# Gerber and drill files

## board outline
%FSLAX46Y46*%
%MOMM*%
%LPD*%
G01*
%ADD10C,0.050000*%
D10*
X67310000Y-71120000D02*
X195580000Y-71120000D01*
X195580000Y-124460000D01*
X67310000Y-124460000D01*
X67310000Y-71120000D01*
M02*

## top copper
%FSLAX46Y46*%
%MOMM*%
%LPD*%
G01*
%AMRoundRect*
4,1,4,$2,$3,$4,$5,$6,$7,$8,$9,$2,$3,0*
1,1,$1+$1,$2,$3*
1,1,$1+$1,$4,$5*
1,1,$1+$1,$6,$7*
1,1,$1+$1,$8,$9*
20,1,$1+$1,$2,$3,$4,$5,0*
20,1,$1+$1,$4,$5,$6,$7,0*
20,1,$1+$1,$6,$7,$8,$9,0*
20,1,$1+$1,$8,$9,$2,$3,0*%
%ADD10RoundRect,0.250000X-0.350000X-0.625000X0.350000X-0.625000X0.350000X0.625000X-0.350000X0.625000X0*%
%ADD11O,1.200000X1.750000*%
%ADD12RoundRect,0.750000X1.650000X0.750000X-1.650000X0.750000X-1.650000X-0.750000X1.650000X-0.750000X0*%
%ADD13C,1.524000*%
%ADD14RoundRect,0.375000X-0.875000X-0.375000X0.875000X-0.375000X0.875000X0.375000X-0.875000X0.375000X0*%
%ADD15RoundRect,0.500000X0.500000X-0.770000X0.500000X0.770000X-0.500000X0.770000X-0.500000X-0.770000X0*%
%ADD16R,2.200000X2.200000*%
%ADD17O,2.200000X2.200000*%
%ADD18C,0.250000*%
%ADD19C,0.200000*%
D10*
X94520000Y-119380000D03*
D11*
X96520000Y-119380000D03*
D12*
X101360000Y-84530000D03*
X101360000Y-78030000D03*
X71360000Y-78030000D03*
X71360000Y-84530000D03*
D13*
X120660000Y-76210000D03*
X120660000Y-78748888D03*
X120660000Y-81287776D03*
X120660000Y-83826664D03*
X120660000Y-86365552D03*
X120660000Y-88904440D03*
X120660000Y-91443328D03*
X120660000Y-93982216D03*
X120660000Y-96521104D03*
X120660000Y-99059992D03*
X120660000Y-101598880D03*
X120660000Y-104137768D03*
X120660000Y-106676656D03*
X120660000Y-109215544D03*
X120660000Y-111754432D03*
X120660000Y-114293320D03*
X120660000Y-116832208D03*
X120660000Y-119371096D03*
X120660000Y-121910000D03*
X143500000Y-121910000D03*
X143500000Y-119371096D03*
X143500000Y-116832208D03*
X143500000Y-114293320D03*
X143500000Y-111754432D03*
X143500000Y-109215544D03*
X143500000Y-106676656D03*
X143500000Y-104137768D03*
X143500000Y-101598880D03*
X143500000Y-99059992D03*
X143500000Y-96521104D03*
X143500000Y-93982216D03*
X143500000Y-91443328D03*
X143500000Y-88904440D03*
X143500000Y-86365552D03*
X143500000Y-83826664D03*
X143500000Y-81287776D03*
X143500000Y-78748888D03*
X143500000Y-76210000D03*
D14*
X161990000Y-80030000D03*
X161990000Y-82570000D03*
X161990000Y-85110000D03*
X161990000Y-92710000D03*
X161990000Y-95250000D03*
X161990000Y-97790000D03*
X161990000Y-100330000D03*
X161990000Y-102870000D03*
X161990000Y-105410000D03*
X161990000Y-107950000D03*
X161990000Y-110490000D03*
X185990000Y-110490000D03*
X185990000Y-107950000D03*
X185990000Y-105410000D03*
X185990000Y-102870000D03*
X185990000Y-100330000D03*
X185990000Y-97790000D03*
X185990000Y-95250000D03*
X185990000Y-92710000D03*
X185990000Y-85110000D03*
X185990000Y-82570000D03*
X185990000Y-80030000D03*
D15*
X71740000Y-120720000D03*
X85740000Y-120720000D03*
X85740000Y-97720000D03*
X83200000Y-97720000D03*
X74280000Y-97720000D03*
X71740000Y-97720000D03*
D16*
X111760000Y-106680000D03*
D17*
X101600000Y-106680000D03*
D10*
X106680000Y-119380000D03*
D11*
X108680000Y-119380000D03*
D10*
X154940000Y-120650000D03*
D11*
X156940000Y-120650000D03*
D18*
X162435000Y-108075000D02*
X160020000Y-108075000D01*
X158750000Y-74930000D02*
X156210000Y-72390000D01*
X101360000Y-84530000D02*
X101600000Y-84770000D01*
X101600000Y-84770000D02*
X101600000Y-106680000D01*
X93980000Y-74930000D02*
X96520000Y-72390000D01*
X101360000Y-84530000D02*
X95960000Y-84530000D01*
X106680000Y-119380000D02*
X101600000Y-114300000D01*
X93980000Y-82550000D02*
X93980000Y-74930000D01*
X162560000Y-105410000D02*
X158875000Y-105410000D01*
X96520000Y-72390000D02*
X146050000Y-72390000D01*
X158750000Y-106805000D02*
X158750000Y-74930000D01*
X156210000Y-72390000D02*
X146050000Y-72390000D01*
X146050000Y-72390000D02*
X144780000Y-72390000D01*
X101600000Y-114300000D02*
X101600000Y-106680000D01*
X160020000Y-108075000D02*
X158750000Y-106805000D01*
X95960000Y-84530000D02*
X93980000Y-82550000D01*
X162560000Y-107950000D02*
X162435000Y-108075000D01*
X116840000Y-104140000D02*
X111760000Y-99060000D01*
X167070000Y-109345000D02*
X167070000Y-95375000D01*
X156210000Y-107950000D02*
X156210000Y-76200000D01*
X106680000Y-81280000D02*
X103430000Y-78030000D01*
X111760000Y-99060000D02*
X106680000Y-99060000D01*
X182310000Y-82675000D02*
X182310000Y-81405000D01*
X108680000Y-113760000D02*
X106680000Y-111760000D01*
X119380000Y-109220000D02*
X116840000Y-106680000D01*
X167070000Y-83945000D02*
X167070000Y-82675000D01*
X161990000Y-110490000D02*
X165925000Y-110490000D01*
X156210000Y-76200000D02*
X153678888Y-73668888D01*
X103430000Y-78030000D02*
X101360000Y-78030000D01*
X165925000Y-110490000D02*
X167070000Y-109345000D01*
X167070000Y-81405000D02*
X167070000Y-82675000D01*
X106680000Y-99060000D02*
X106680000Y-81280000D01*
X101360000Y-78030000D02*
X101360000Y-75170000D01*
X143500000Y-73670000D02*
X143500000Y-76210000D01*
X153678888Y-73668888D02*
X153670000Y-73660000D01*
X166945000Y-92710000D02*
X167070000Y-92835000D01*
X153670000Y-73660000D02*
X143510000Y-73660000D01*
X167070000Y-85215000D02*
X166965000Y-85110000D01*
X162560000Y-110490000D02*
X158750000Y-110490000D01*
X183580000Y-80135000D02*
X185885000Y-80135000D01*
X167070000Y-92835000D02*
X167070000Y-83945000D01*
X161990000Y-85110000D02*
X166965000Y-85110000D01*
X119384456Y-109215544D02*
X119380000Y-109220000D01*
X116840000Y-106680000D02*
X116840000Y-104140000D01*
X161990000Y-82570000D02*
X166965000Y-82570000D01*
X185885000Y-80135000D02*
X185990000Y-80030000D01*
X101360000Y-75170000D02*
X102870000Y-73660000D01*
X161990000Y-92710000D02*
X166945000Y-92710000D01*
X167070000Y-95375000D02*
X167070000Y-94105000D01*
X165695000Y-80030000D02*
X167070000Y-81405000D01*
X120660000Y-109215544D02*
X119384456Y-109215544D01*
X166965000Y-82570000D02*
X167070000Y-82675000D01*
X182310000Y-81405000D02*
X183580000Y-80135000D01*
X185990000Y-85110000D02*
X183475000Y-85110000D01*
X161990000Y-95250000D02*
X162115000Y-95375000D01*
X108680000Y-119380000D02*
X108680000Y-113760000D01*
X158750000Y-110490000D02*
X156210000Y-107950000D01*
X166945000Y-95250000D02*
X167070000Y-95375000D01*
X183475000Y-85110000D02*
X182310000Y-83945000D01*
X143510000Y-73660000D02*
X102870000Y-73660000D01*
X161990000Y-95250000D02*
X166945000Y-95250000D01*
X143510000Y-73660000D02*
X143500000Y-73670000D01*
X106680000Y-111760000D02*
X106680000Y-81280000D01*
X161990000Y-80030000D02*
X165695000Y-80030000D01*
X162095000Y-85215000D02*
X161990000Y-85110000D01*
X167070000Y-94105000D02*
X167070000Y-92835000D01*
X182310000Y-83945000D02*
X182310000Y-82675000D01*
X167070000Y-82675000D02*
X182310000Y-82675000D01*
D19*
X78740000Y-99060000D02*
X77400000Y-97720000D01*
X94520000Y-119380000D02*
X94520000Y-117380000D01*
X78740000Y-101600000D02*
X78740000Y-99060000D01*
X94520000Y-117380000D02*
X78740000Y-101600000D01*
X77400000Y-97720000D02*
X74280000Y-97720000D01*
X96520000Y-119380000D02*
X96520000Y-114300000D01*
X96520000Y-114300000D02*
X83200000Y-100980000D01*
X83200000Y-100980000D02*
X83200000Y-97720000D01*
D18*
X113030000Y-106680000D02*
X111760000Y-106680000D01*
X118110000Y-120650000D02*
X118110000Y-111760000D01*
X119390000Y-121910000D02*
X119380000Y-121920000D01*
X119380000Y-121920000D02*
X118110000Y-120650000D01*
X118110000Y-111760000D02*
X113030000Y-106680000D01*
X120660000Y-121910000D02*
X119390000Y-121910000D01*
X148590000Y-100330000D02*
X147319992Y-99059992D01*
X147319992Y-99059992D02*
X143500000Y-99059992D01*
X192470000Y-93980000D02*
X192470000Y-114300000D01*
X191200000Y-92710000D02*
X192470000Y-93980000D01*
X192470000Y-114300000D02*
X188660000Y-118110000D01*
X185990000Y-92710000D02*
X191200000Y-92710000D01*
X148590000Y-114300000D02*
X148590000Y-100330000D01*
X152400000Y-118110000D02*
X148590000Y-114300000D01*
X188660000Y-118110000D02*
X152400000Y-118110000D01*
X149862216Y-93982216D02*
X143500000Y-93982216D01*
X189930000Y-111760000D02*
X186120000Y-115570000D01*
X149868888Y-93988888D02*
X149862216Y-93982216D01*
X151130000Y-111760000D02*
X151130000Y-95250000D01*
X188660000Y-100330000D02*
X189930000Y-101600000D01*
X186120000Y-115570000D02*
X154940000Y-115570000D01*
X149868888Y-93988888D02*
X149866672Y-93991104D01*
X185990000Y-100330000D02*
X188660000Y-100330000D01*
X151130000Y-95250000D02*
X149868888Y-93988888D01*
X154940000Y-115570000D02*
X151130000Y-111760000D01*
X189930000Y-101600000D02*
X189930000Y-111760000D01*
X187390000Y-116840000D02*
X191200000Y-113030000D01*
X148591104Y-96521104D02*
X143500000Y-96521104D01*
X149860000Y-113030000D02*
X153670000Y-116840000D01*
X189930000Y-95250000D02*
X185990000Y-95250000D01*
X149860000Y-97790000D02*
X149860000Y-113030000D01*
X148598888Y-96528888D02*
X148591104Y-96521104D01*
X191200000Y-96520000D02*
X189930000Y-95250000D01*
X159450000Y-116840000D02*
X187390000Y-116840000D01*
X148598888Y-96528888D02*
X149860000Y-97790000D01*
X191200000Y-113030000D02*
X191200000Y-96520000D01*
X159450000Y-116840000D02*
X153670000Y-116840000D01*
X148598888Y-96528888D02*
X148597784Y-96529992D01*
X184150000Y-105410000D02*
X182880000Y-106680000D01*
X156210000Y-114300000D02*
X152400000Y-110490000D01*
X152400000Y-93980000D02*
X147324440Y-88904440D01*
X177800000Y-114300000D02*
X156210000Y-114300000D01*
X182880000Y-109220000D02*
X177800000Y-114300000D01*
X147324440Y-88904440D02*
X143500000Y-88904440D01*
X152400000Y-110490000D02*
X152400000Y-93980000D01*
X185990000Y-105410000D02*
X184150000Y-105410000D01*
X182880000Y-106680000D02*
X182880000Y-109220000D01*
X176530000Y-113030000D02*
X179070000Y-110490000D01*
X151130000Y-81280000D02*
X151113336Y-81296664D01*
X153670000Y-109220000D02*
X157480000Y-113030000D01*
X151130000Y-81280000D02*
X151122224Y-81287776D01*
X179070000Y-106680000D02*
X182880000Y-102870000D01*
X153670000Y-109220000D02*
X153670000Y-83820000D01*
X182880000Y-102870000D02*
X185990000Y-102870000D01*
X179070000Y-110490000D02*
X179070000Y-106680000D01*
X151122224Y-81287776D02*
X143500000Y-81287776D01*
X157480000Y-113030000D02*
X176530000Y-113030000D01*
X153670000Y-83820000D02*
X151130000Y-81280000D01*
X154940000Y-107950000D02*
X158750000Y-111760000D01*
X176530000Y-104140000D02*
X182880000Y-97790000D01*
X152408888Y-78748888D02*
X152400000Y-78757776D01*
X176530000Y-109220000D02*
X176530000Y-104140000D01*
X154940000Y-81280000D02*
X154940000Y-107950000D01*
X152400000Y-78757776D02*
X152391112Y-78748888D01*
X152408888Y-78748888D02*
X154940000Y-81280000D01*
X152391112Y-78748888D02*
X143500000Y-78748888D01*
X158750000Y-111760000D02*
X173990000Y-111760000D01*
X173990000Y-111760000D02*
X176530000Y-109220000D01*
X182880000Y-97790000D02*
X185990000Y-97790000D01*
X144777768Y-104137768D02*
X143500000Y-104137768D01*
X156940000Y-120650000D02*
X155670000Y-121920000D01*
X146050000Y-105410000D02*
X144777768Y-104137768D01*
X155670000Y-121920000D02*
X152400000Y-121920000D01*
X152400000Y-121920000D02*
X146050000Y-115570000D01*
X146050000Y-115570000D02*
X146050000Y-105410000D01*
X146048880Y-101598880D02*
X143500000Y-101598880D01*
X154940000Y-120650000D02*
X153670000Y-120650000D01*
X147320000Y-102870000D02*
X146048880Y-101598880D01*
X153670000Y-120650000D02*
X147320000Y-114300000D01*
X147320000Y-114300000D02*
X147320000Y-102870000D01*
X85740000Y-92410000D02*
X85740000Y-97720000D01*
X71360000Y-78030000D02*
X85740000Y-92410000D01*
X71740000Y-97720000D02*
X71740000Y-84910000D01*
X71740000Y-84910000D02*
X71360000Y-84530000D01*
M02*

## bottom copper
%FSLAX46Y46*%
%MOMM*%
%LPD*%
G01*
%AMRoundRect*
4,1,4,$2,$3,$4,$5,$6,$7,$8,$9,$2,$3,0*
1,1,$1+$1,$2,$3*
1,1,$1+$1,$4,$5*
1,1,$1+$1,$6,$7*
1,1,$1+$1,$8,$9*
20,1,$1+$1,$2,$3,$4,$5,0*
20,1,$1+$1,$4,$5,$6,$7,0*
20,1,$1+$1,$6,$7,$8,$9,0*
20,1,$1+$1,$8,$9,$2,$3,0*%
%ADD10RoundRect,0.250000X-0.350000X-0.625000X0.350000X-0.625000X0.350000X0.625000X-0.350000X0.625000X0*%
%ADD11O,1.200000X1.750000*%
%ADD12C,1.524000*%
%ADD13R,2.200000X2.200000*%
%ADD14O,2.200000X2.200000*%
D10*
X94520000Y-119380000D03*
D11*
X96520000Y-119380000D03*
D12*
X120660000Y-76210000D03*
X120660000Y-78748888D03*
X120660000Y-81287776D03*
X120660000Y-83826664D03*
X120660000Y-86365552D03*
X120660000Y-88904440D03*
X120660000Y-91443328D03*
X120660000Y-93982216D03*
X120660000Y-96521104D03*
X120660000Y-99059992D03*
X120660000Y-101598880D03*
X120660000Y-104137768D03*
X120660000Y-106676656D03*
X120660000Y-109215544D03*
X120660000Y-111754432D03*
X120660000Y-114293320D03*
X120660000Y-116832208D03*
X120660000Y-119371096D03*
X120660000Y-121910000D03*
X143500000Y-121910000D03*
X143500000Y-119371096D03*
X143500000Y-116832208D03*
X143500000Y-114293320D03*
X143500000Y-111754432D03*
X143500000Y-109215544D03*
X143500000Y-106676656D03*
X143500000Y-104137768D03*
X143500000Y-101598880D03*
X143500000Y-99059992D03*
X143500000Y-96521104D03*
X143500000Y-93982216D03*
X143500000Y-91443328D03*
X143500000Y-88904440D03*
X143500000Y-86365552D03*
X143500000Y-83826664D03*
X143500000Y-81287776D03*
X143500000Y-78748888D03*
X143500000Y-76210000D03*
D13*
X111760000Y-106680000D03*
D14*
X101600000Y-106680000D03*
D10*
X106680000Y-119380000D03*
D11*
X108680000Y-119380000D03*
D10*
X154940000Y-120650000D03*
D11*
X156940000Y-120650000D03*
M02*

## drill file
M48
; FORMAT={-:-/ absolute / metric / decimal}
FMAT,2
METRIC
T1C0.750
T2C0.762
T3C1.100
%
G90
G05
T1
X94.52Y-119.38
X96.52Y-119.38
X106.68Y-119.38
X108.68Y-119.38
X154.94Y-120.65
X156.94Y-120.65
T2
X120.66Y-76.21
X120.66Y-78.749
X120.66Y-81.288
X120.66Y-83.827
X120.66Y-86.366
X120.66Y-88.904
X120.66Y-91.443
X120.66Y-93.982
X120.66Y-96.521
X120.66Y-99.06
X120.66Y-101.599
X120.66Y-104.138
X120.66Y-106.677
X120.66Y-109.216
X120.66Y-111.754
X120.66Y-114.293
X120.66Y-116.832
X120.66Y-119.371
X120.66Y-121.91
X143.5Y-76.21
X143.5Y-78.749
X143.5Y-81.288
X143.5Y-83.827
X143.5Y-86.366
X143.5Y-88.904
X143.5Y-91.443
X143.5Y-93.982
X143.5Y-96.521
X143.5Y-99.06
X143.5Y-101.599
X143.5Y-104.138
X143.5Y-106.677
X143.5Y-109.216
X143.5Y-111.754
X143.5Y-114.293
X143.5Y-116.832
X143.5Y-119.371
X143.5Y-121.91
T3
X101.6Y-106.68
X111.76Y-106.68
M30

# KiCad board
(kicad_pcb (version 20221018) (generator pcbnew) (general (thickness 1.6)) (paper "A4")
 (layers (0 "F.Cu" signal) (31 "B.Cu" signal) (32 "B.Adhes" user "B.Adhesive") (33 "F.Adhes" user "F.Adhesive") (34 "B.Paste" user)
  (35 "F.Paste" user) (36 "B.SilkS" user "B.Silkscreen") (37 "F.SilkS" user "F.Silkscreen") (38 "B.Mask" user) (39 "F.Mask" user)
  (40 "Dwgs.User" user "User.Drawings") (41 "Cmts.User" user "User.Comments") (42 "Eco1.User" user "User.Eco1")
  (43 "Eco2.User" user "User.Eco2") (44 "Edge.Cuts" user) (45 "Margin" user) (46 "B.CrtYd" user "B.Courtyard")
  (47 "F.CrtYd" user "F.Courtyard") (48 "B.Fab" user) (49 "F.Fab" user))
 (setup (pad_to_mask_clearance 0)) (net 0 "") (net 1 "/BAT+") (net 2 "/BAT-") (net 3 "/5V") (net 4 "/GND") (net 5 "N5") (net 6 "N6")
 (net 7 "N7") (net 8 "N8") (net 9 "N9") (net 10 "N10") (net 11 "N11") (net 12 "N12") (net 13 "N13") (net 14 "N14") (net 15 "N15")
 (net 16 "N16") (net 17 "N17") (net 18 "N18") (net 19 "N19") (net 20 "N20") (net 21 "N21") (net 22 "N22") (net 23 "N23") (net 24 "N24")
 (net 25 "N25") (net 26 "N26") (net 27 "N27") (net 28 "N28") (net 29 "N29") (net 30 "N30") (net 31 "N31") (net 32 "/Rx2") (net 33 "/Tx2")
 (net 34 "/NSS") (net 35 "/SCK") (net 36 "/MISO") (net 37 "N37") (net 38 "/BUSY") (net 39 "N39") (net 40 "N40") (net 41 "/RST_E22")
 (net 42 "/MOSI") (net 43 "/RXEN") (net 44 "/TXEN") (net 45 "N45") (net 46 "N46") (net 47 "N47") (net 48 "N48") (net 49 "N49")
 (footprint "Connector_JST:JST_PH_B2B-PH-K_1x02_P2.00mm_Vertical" (layer "F.Cu") (at 94.52 119.38)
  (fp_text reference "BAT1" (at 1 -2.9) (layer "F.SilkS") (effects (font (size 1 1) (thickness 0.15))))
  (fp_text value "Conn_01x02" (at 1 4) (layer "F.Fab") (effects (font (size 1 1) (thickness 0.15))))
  (pad "1" thru_hole roundrect (at 0 0) (size 1.2 1.75) (drill 0.75) (layers "*.Cu" "*.Mask") (roundrect_rratio 0.208333) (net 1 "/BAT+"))
  (pad "2" thru_hole oval (at 2 0) (size 1.2 1.75) (drill 0.75) (layers "*.Cu" "*.Mask") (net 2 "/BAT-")))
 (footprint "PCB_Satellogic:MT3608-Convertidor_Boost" (layer "F.Cu") (at 86.36 81.28 180)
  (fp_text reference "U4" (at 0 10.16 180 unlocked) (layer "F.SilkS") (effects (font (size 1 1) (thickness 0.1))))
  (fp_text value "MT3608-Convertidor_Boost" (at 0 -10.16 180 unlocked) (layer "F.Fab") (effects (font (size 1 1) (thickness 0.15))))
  (pad "1" smd roundrect (at -15 -3.25 180) (size 4.8 3) (layers "F.Cu" "F.Paste" "F.Mask") (roundrect_rratio 0.25) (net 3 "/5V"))
  (pad "2" smd roundrect (at -15 3.25 180) (size 4.8 3) (layers "F.Cu" "F.Paste" "F.Mask") (roundrect_rratio 0.25) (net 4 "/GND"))
  (pad "3" smd roundrect (at 15 3.25 180) (size 4.8 3) (layers "F.Cu" "F.Paste" "F.Mask") (roundrect_rratio 0.25) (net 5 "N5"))
  (pad "4" smd roundrect (at 15 -3.25 180) (size 4.8 3) (layers "F.Cu" "F.Paste" "F.Mask") (roundrect_rratio 0.25) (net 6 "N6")))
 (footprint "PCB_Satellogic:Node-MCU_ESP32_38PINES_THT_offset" (layer "F.Cu") (at 132.08 99.06)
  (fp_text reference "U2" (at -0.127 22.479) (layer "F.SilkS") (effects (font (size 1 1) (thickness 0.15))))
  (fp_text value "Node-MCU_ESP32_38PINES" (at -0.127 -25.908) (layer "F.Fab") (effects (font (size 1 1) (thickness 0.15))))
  (pad "1" thru_hole circle (at -11.42 -22.85) (size 1.524 1.524) (drill 0.762) (layers "*.Cu" "*.Mask") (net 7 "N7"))
  (pad "2" thru_hole circle (at -11.42 -20.311112) (size 1.524 1.524) (drill 0.762) (layers "*.Cu" "*.Mask") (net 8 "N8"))
  (pad "3" thru_hole circle (at -11.42 -17.772224) (size 1.524 1.524) (drill 0.762) (layers "*.Cu" "*.Mask") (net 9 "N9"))
  (pad "4" thru_hole circle (at -11.42 -15.233336) (size 1.524 1.524) (drill 0.762) (layers "*.Cu" "*.Mask") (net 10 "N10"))
  (pad "5" thru_hole circle (at -11.42 -12.694448) (size 1.524 1.524) (drill 0.762) (layers "*.Cu" "*.Mask") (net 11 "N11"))
  (pad "6" thru_hole circle (at -11.42 -10.15556) (size 1.524 1.524) (drill 0.762) (layers "*.Cu" "*.Mask") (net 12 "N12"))
  (pad "7" thru_hole circle (at -11.42 -7.616672) (size 1.524 1.524) (drill 0.762) (layers "*.Cu" "*.Mask") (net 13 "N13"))
  (pad "8" thru_hole circle (at -11.42 -5.077784) (size 1.524 1.524) (drill 0.762) (layers "*.Cu" "*.Mask") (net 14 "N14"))
  (pad "9" thru_hole circle (at -11.42 -2.538896) (size 1.524 1.524) (drill 0.762) (layers "*.Cu" "*.Mask") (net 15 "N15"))
  (pad "10" thru_hole circle (at -11.42 -0.000008) (size 1.524 1.524) (drill 0.762) (layers "*.Cu" "*.Mask") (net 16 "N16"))
  (pad "11" thru_hole circle (at -11.42 2.53888) (size 1.524 1.524) (drill 0.762) (layers "*.Cu" "*.Mask") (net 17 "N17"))
  (pad "12" thru_hole circle (at -11.42 5.077768) (size 1.524 1.524) (drill 0.762) (layers "*.Cu" "*.Mask") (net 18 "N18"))
  (pad "13" thru_hole circle (at -11.42 7.616656) (size 1.524 1.524) (drill 0.762) (layers "*.Cu" "*.Mask") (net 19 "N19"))
  (pad "14" thru_hole circle (at -11.42 10.155544) (size 1.524 1.524) (drill 0.762) (layers "*.Cu" "*.Mask") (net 4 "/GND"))
  (pad "15" thru_hole circle (at -11.42 12.694432) (size 1.524 1.524) (drill 0.762) (layers "*.Cu" "*.Mask") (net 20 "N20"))
  (pad "16" thru_hole circle (at -11.42 15.23332) (size 1.524 1.524) (drill 0.762) (layers "*.Cu" "*.Mask") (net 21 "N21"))
  (pad "17" thru_hole circle (at -11.42 17.772208) (size 1.524 1.524) (drill 0.762) (layers "*.Cu" "*.Mask") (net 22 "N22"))
  (pad "18" thru_hole circle (at -11.42 20.311096) (size 1.524 1.524) (drill 0.762) (layers "*.Cu" "*.Mask") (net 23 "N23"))
  (pad "19" thru_hole circle (at -11.42 22.85) (size 1.524 1.524) (drill 0.762) (layers "*.Cu" "*.Mask") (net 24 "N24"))
  (pad "20" thru_hole circle (at 11.42 22.85) (size 1.524 1.524) (drill 0.762) (layers "*.Cu" "*.Mask") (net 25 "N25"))
  (pad "21" thru_hole circle (at 11.42 20.311096) (size 1.524 1.524) (drill 0.762) (layers "*.Cu" "*.Mask") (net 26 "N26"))
  (pad "22" thru_hole circle (at 11.42 17.772208) (size 1.524 1.524) (drill 0.762) (layers "*.Cu" "*.Mask") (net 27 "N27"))
  (pad "23" thru_hole circle (at 11.42 15.23332) (size 1.524 1.524) (drill 0.762) (layers "*.Cu" "*.Mask") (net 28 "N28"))
  (pad "24" thru_hole circle (at 11.42 12.694432) (size 1.524 1.524) (drill 0.762) (layers "*.Cu" "*.Mask") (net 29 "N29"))
  (pad "25" thru_hole circle (at 11.42 10.155544) (size 1.524 1.524) (drill 0.762) (layers "*.Cu" "*.Mask") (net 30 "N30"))
  (pad "26" thru_hole circle (at 11.42 7.616656) (size 1.524 1.524) (drill 0.762) (layers "*.Cu" "*.Mask") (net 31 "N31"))
  (pad "27" thru_hole circle (at 11.42 5.077768) (size 1.524 1.524) (drill 0.762) (layers "*.Cu" "*.Mask") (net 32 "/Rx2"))
  (pad "28" thru_hole circle (at 11.42 2.53888) (size 1.524 1.524) (drill 0.762) (layers "*.Cu" "*.Mask") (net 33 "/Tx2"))
  (pad "29" thru_hole circle (at 11.42 -0.000008) (size 1.524 1.524) (drill 0.762) (layers "*.Cu" "*.Mask") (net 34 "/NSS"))
  (pad "30" thru_hole circle (at 11.42 -2.538896) (size 1.524 1.524) (drill 0.762) (layers "*.Cu" "*.Mask") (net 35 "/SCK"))
  (pad "31" thru_hole circle (at 11.42 -5.077784) (size 1.524 1.524) (drill 0.762) (layers "*.Cu" "*.Mask") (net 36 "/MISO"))
  (pad "32" thru_hole circle (at 11.42 -7.616672) (size 1.524 1.524) (drill 0.762) (layers "*.Cu" "*.Mask") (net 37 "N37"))
  (pad "33" thru_hole circle (at 11.42 -10.15556) (size 1.524 1.524) (drill 0.762) (layers "*.Cu" "*.Mask") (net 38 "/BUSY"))
  (pad "34" thru_hole circle (at 11.42 -12.694448) (size 1.524 1.524) (drill 0.762) (layers "*.Cu" "*.Mask") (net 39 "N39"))
  (pad "35" thru_hole circle (at 11.42 -15.233336) (size 1.524 1.524) (drill 0.762) (layers "*.Cu" "*.Mask") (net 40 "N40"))
  (pad "36" thru_hole circle (at 11.42 -17.772224) (size 1.524 1.524) (drill 0.762) (layers "*.Cu" "*.Mask") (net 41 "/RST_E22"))
  (pad "37" thru_hole circle (at 11.42 -20.311112) (size 1.524 1.524) (drill 0.762) (layers "*.Cu" "*.Mask") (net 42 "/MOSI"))
  (pad "38" thru_hole circle (at 11.42 -22.85) (size 1.524 1.524) (drill 0.762) (layers "*.Cu" "*.Mask") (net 4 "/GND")))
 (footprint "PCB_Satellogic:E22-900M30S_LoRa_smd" (layer "F.Cu") (at 173.99 94.105)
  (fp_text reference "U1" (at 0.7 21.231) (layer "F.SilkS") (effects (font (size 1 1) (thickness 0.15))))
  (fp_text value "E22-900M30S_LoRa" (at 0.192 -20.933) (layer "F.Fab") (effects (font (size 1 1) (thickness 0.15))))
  (pad "1" smd roundrect (at -12 -14.075) (size 2.5 1.5) (layers "F.Cu" "F.Paste" "F.Mask") (roundrect_rratio 0.25) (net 4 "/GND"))
  (pad "2" smd roundrect (at -12 -11.535) (size 2.5 1.5) (layers "F.Cu" "F.Paste" "F.Mask") (roundrect_rratio 0.25) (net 4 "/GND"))
  (pad "3" smd roundrect (at -12 -8.995) (size 2.5 1.5) (layers "F.Cu" "F.Paste" "F.Mask") (roundrect_rratio 0.25) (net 4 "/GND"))
  (pad "4" smd roundrect (at -12 -1.395) (size 2.5 1.5) (layers "F.Cu" "F.Paste" "F.Mask") (roundrect_rratio 0.25) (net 4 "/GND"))
  (pad "5" smd roundrect (at -12 1.145) (size 2.5 1.5) (layers "F.Cu" "F.Paste" "F.Mask") (roundrect_rratio 0.25) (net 4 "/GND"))
  (pad "6" smd roundrect (at -12 3.685) (size 2.5 1.5) (layers "F.Cu" "F.Paste" "F.Mask") (roundrect_rratio 0.25) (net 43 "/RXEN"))
  (pad "7" smd roundrect (at -12 6.225) (size 2.5 1.5) (layers "F.Cu" "F.Paste" "F.Mask") (roundrect_rratio 0.25) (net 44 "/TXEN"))
  (pad "8" smd roundrect (at -12 8.765) (size 2.5 1.5) (layers "F.Cu" "F.Paste" "F.Mask") (roundrect_rratio 0.25) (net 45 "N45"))
  (pad "9" smd roundrect (at -12 11.305) (size 2.5 1.5) (layers "F.Cu" "F.Paste" "F.Mask") (roundrect_rratio 0.25) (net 3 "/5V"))
  (pad "10" smd roundrect (at -12 13.845) (size 2.5 1.5) (layers "F.Cu" "F.Paste" "F.Mask") (roundrect_rratio 0.25) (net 3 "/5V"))
  (pad "11" smd roundrect (at -12 16.385) (size 2.5 1.5) (layers "F.Cu" "F.Paste" "F.Mask") (roundrect_rratio 0.25) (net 4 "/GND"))
  (pad "12" smd roundrect (at 12 16.385) (size 2.5 1.5) (layers "F.Cu" "F.Paste" "F.Mask") (roundrect_rratio 0.25) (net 4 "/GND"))
  (pad "13" smd roundrect (at 12 13.845) (size 2.5 1.5) (layers "F.Cu" "F.Paste" "F.Mask") (roundrect_rratio 0.25) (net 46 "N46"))
  (pad "14" smd roundrect (at 12 11.305) (size 2.5 1.5) (layers "F.Cu" "F.Paste" "F.Mask") (roundrect_rratio 0.25) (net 38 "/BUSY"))
  (pad "15" smd roundrect (at 12 8.765) (size 2.5 1.5) (layers "F.Cu" "F.Paste" "F.Mask") (roundrect_rratio 0.25) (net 41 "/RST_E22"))
  (pad "16" smd roundrect (at 12 6.225) (size 2.5 1.5) (layers "F.Cu" "F.Paste" "F.Mask") (roundrect_rratio 0.25) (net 36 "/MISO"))
  (pad "17" smd roundrect (at 12 3.685) (size 2.5 1.5) (layers "F.Cu" "F.Paste" "F.Mask") (roundrect_rratio 0.25) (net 42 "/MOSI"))
  (pad "18" smd roundrect (at 12 1.145) (size 2.5 1.5) (layers "F.Cu" "F.Paste" "F.Mask") (roundrect_rratio 0.25) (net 35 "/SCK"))
  (pad "19" smd roundrect (at 12 -1.395) (size 2.5 1.5) (layers "F.Cu" "F.Paste" "F.Mask") (roundrect_rratio 0.25) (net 34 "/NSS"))
  (pad "20" smd roundrect (at 12 -8.995) (size 2.5 1.5) (layers "F.Cu" "F.Paste" "F.Mask") (roundrect_rratio 0.25) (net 4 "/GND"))
  (pad "21" smd roundrect (at 12 -11.535) (size 2.5 1.5) (layers "F.Cu" "F.Paste" "F.Mask") (roundrect_rratio 0.25) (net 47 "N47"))
  (pad "22" smd roundrect (at 12 -14.075) (size 2.5 1.5) (layers "F.Cu" "F.Paste" "F.Mask") (roundrect_rratio 0.25) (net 4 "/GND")))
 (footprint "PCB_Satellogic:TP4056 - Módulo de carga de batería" (layer "F.Cu") (at 78.74 109.22 90)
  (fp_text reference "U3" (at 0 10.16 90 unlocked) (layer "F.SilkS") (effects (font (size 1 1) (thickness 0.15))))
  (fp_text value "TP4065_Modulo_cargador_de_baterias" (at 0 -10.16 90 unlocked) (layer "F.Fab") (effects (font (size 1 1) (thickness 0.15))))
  (pad "1" smd roundrect (at -11.5 -7 90) (size 2.54 2) (layers "F.Cu" "F.Paste" "F.Mask") (roundrect_rratio 0.25) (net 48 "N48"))
  (pad "2" smd roundrect (at -11.5 7 90) (size 2.54 2) (layers "F.Cu" "F.Paste" "F.Mask") (roundrect_rratio 0.25) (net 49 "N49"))
  (pad "3" smd roundrect (at 11.5 7 90) (size 2.54 2) (layers "F.Cu" "F.Paste" "F.Mask") (roundrect_rratio 0.25) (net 5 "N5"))
  (pad "4" smd roundrect (at 11.5 4.46 90) (size 2.54 2) (layers "F.Cu" "F.Paste" "F.Mask") (roundrect_rratio 0.25) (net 2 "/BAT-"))
  (pad "5" smd roundrect (at 11.5 -4.46 90) (size 2.54 2) (layers "F.Cu" "F.Paste" "F.Mask") (roundrect_rratio 0.25) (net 1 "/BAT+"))
  (pad "6" smd roundrect (at 11.5 -7 90) (size 2.54 2) (layers "F.Cu" "F.Paste" "F.Mask") (roundrect_rratio 0.25) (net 6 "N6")))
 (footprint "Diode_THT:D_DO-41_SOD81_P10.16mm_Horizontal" (layer "F.Cu") (at 111.76 106.68 180)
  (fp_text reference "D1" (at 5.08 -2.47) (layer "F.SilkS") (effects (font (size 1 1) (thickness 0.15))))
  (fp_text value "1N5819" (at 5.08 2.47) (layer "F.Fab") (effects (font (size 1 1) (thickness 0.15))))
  (pad "1" thru_hole rect (at 0 0 180) (size 2.2 2.2) (drill 1.1) (layers "*.Cu" "*.Mask") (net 24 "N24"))
  (pad "2" thru_hole oval (at 10.16 0 180) (size 2.2 2.2) (drill 1.1) (layers "*.Cu" "*.Mask") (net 3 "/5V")))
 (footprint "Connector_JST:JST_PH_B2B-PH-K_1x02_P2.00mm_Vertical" (layer "F.Cu") (at 106.68 119.38)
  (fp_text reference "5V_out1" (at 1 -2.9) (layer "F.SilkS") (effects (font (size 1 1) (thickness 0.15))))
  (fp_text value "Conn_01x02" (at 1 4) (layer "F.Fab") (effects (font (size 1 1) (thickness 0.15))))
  (pad "1" thru_hole roundrect (at 0 0) (size 1.2 1.75) (drill 0.75) (layers "*.Cu" "*.Mask") (roundrect_rratio 0.208333) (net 3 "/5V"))
  (pad "2" thru_hole oval (at 2 0) (size 1.2 1.75) (drill 0.75) (layers "*.Cu" "*.Mask") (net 4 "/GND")))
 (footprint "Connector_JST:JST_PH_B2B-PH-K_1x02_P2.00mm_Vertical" (layer "F.Cu") (at 154.94 120.65)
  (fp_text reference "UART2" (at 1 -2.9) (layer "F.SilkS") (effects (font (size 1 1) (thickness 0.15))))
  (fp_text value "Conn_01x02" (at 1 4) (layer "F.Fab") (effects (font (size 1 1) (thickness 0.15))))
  (pad "1" thru_hole roundrect (at 0 0) (size 1.2 1.75) (drill 0.75) (layers "*.Cu" "*.Mask") (roundrect_rratio 0.208333) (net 33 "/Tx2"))
  (pad "2" thru_hole oval (at 2 0) (size 1.2 1.75) (drill 0.75) (layers "*.Cu" "*.Mask") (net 32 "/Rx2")))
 (gr_rect (start 67.31 71.12) (end 195.58 124.46) (stroke (width 0.05) (type default)) (fill none) (layer "Edge.Cuts"))
 (segment (start 162.435 108.075) (end 160.02 108.075) (width 0.25) (layer "F.Cu") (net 3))
 (segment (start 158.75 74.93) (end 156.21 72.39) (width 0.25) (layer "F.Cu") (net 3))
 (segment (start 101.36 84.53) (end 101.6 84.77) (width 0.25) (layer "F.Cu") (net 3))
 (segment (start 101.6 84.77) (end 101.6 106.68) (width 0.25) (layer "F.Cu") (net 3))
 (segment (start 93.98 74.93) (end 96.52 72.39) (width 0.25) (layer "F.Cu") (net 3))
 (segment (start 101.36 84.53) (end 95.96 84.53) (width 0.25) (layer "F.Cu") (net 3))
 (segment (start 106.68 119.38) (end 101.6 114.3) (width 0.25) (layer "F.Cu") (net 3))
 (segment (start 93.98 82.55) (end 93.98 74.93) (width 0.25) (layer "F.Cu") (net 3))
 (segment (start 162.56 105.41) (end 158.875 105.41) (width 0.25) (layer "F.Cu") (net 3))
 (segment (start 96.52 72.39) (end 146.05 72.39) (width 0.25) (layer "F.Cu") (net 3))
 (segment (start 158.75 106.805) (end 158.75 74.93) (width 0.25) (layer "F.Cu") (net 3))
 (segment (start 156.21 72.39) (end 146.05 72.39) (width 0.25) (layer "F.Cu") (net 3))
 (segment (start 146.05 72.39) (end 144.78 72.39) (width 0.25) (layer "F.Cu") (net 3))
 (segment (start 101.6 114.3) (end 101.6 106.68) (width 0.25) (layer "F.Cu") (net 3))
 (segment (start 160.02 108.075) (end 158.75 106.805) (width 0.25) (layer "F.Cu") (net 3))
 (segment (start 95.96 84.53) (end 93.98 82.55) (width 0.25) (layer "F.Cu") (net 3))
 (segment (start 162.56 107.95) (end 162.435 108.075) (width 0.25) (layer "F.Cu") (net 3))
 (segment (start 116.84 104.14) (end 111.76 99.06) (width 0.25) (layer "F.Cu") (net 4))
 (segment (start 167.07 109.345) (end 167.07 95.375) (width 0.25) (layer "F.Cu") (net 4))
 (segment (start 156.21 107.95) (end 156.21 76.2) (width 0.25) (layer "F.Cu") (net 4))
 (segment (start 106.68 81.28) (end 103.43 78.03) (width 0.25) (layer "F.Cu") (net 4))
 (segment (start 111.76 99.06) (end 106.68 99.06) (width 0.25) (layer "F.Cu") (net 4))
 (segment (start 182.31 82.675) (end 182.31 81.405) (width 0.25) (layer "F.Cu") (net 4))
 (segment (start 108.68 113.76) (end 106.68 111.76) (width 0.25) (layer "F.Cu") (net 4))
 (segment (start 119.38 109.22) (end 116.84 106.68) (width 0.25) (layer "F.Cu") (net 4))
 (segment (start 167.07 83.945) (end 167.07 82.675) (width 0.25) (layer "F.Cu") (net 4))
 (segment (start 161.99 110.49) (end 165.925 110.49) (width 0.25) (layer "F.Cu") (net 4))
 (segment (start 156.21 76.2) (end 153.678888 73.668888) (width 0.25) (layer "F.Cu") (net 4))
 (segment (start 103.43 78.03) (end 101.36 78.03) (width 0.25) (layer "F.Cu") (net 4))
 (segment (start 165.925 110.49) (end 167.07 109.345) (width 0.25) (layer "F.Cu") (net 4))
 (segment (start 167.07 81.405) (end 167.07 82.675) (width 0.25) (layer "F.Cu") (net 4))
 (segment (start 106.68 99.06) (end 106.68 81.28) (width 0.25) (layer "F.Cu") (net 4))
 (segment (start 101.36 78.03) (end 101.36 75.17) (width 0.25) (layer "F.Cu") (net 4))
 (segment (start 143.5 73.67) (end 143.5 76.21) (width 0.25) (layer "F.Cu") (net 4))
 (segment (start 153.678888 73.668888) (end 153.67 73.66) (width 0.25) (layer "F.Cu") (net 4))
 (segment (start 166.945 92.71) (end 167.07 92.835) (width 0.25) (layer "F.Cu") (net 4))
 (segment (start 153.67 73.66) (end 143.51 73.66) (width 0.25) (layer "F.Cu") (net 4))
 (segment (start 167.07 85.215) (end 166.965 85.11) (width 0.25) (layer "F.Cu") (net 4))
 (segment (start 162.56 110.49) (end 158.75 110.49) (width 0.25) (layer "F.Cu") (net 4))
 (segment (start 183.58 80.135) (end 185.885 80.135) (width 0.25) (layer "F.Cu") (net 4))
 (segment (start 167.07 92.835) (end 167.07 83.945) (width 0.25) (layer "F.Cu") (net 4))
 (segment (start 161.99 85.11) (end 166.965 85.11) (width 0.25) (layer "F.Cu") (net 4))
 (segment (start 119.384456 109.215544) (end 119.38 109.22) (width 0.25) (layer "F.Cu") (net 4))
 (segment (start 116.84 106.68) (end 116.84 104.14) (width 0.25) (layer "F.Cu") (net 4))
 (segment (start 161.99 82.57) (end 166.965 82.57) (width 0.25) (layer "F.Cu") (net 4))
 (segment (start 185.885 80.135) (end 185.99 80.03) (width 0.25) (layer "F.Cu") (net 4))
 (segment (start 101.36 75.17) (end 102.87 73.66) (width 0.25) (layer "F.Cu") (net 4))
 (segment (start 161.99 92.71) (end 166.945 92.71) (width 0.25) (layer "F.Cu") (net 4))
 (segment (start 167.07 95.375) (end 167.07 94.105) (width 0.25) (layer "F.Cu") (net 4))
 (segment (start 165.695 80.03) (end 167.07 81.405) (width 0.25) (layer "F.Cu") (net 4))
 (segment (start 120.66 109.215544) (end 119.384456 109.215544) (width 0.25) (layer "F.Cu") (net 4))
 (segment (start 166.965 82.57) (end 167.07 82.675) (width 0.25) (layer "F.Cu") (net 4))
 (segment (start 182.31 81.405) (end 183.58 80.135) (width 0.25) (layer "F.Cu") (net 4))
 (segment (start 185.99 85.11) (end 183.475 85.11) (width 0.25) (layer "F.Cu") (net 4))
 (segment (start 161.99 95.25) (end 162.115 95.375) (width 0.25) (layer "F.Cu") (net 4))
 (segment (start 108.68 119.38) (end 108.68 113.76) (width 0.25) (layer "F.Cu") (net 4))
 (segment (start 158.75 110.49) (end 156.21 107.95) (width 0.25) (layer "F.Cu") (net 4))
 (segment (start 166.945 95.25) (end 167.07 95.375) (width 0.25) (layer "F.Cu") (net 4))
 (segment (start 183.475 85.11) (end 182.31 83.945) (width 0.25) (layer "F.Cu") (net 4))
 (segment (start 143.51 73.66) (end 102.87 73.66) (width 0.25) (layer "F.Cu") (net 4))
 (segment (start 161.99 95.25) (end 166.945 95.25) (width 0.25) (layer "F.Cu") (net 4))
 (segment (start 143.51 73.66) (end 143.5 73.67) (width 0.25) (layer "F.Cu") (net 4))
 (segment (start 106.68 111.76) (end 106.68 81.28) (width 0.25) (layer "F.Cu") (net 4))
 (segment (start 161.99 80.03) (end 165.695 80.03) (width 0.25) (layer "F.Cu") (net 4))
 (segment (start 162.095 85.215) (end 161.99 85.11) (width 0.25) (layer "F.Cu") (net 4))
 (segment (start 167.07 94.105) (end 167.07 92.835) (width 0.25) (layer "F.Cu") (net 4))
 (segment (start 182.31 83.945) (end 182.31 82.675) (width 0.25) (layer "F.Cu") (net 4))
 (segment (start 167.07 82.675) (end 182.31 82.675) (width 0.25) (layer "F.Cu") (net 4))
 (segment (start 78.74 99.06) (end 77.4 97.72) (width 0.2) (layer "F.Cu") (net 1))
 (segment (start 94.52 119.38) (end 94.52 117.38) (width 0.2) (layer "F.Cu") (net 1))
 (segment (start 78.74 101.6) (end 78.74 99.06) (width 0.2) (layer "F.Cu") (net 1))
 (segment (start 94.52 117.38) (end 78.74 101.6) (width 0.2) (layer "F.Cu") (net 1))
 (segment (start 77.4 97.72) (end 74.28 97.72) (width 0.2) (layer "F.Cu") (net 1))
 (segment (start 96.52 119.38) (end 96.52 114.3) (width 0.2) (layer "F.Cu") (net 2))
 (segment (start 96.52 114.3) (end 83.2 100.98) (width 0.2) (layer "F.Cu") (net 2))
 (segment (start 83.2 100.98) (end 83.2 97.72) (width 0.2) (layer "F.Cu") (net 2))
 (segment (start 113.03 106.68) (end 111.76 106.68) (width 0.25) (layer "F.Cu") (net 24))
 (segment (start 118.11 120.65) (end 118.11 111.76) (width 0.25) (layer "F.Cu") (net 24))
 (segment (start 119.39 121.91) (end 119.38 121.92) (width 0.25) (layer "F.Cu") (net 24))
 (segment (start 119.38 121.92) (end 118.11 120.65) (width 0.25) (layer "F.Cu") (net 24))
 (segment (start 118.11 111.76) (end 113.03 106.68) (width 0.25) (layer "F.Cu") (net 24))
 (segment (start 120.66 121.91) (end 119.39 121.91) (width 0.25) (layer "F.Cu") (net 24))
 (segment (start 148.59 100.33) (end 147.319992 99.059992) (width 0.25) (layer "F.Cu") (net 34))
 (segment (start 147.319992 99.059992) (end 143.5 99.059992) (width 0.25) (layer "F.Cu") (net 34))
 (segment (start 192.47 93.98) (end 192.47 114.3) (width 0.25) (layer "F.Cu") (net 34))
 (segment (start 191.2 92.71) (end 192.47 93.98) (width 0.25) (layer "F.Cu") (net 34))
 (segment (start 192.47 114.3) (end 188.66 118.11) (width 0.25) (layer "F.Cu") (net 34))
 (segment (start 185.99 92.71) (end 191.2 92.71) (width 0.25) (layer "F.Cu") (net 34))
 (segment (start 148.59 114.3) (end 148.59 100.33) (width 0.25) (layer "F.Cu") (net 34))
 (segment (start 152.4 118.11) (end 148.59 114.3) (width 0.25) (layer "F.Cu") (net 34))
 (segment (start 188.66 118.11) (end 152.4 118.11) (width 0.25) (layer "F.Cu") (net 34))
 (segment (start 149.862216 93.982216) (end 143.5 93.982216) (width 0.25) (layer "F.Cu") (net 36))
 (segment (start 189.93 111.76) (end 186.12 115.57) (width 0.25) (layer "F.Cu") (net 36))
 (segment (start 149.868888 93.988888) (end 149.862216 93.982216) (width 0.25) (layer "F.Cu") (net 36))
 (segment (start 151.13 111.76) (end 151.13 95.25) (width 0.25) (layer "F.Cu") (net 36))
 (segment (start 188.66 100.33) (end 189.93 101.6) (width 0.25) (layer "F.Cu") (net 36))
 (segment (start 186.12 115.57) (end 154.94 115.57) (width 0.25) (layer "F.Cu") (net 36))
 (segment (start 149.868888 93.988888) (end 149.866672 93.991104) (width 0.25) (layer "F.Cu") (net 36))
 (segment (start 185.99 100.33) (end 188.66 100.33) (width 0.25) (layer "F.Cu") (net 36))
 (segment (start 151.13 95.25) (end 149.868888 93.988888) (width 0.25) (layer "F.Cu") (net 36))
 (segment (start 154.94 115.57) (end 151.13 111.76) (width 0.25) (layer "F.Cu") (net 36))
 (segment (start 189.93 101.6) (end 189.93 111.76) (width 0.25) (layer "F.Cu") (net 36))
 (segment (start 187.39 116.84) (end 191.2 113.03) (width 0.25) (layer "F.Cu") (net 35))
 (segment (start 148.591104 96.521104) (end 143.5 96.521104) (width 0.25) (layer "F.Cu") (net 35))
 (segment (start 149.86 113.03) (end 153.67 116.84) (width 0.25) (layer "F.Cu") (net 35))
 (segment (start 189.93 95.25) (end 185.99 95.25) (width 0.25) (layer "F.Cu") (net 35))
 (segment (start 149.86 97.79) (end 149.86 113.03) (width 0.25) (layer "F.Cu") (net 35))
 (segment (start 148.598888 96.528888) (end 148.591104 96.521104) (width 0.25) (layer "F.Cu") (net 35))
 (segment (start 191.2 96.52) (end 189.93 95.25) (width 0.25) (layer "F.Cu") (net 35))
 (segment (start 159.45 116.84) (end 187.39 116.84) (width 0.25) (layer "F.Cu") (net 35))
 (segment (start 148.598888 96.528888) (end 149.86 97.79) (width 0.25) (layer "F.Cu") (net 35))
 (segment (start 191.2 113.03) (end 191.2 96.52) (width 0.25) (layer "F.Cu") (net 35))
 (segment (start 159.45 116.84) (end 153.67 116.84) (width 0.25) (layer "F.Cu") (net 35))
 (segment (start 148.598888 96.528888) (end 148.597784 96.529992) (width 0.25) (layer "F.Cu") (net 35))
 (segment (start 184.15 105.41) (end 182.88 106.68) (width 0.25) (layer "F.Cu") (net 38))
 (segment (start 156.21 114.3) (end 152.4 110.49) (width 0.25) (layer "F.Cu") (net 38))
 (segment (start 152.4 93.98) (end 147.32444 88.90444) (width 0.25) (layer "F.Cu") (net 38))
 (segment (start 177.8 114.3) (end 156.21 114.3) (width 0.25) (layer "F.Cu") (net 38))
 (segment (start 182.88 109.22) (end 177.8 114.3) (width 0.25) (layer "F.Cu") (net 38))
 (segment (start 147.32444 88.90444) (end 143.5 88.90444) (width 0.25) (layer "F.Cu") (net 38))
 (segment (start 152.4 110.49) (end 152.4 93.98) (width 0.25) (layer "F.Cu") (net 38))
 (segment (start 185.99 105.41) (end 184.15 105.41) (width 0.25) (layer "F.Cu") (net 38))
 (segment (start 182.88 106.68) (end 182.88 109.22) (width 0.25) (layer "F.Cu") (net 38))
 (segment (start 176.53 113.03) (end 179.07 110.49) (width 0.25) (layer "F.Cu") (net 41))
 (segment (start 151.13 81.28) (end 151.113336 81.296664) (width 0.25) (layer "F.Cu") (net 41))
 (segment (start 153.67 109.22) (end 157.48 113.03) (width 0.25) (layer "F.Cu") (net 41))
 (segment (start 151.13 81.28) (end 151.122224 81.287776) (width 0.25) (layer "F.Cu") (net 41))
 (segment (start 179.07 106.68) (end 182.88 102.87) (width 0.25) (layer "F.Cu") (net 41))
 (segment (start 153.67 109.22) (end 153.67 83.82) (width 0.25) (layer "F.Cu") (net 41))
 (segment (start 182.88 102.87) (end 185.99 102.87) (width 0.25) (layer "F.Cu") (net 41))
 (segment (start 179.07 110.49) (end 179.07 106.68) (width 0.25) (layer "F.Cu") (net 41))
 (segment (start 151.122224 81.287776) (end 143.5 81.287776) (width 0.25) (layer "F.Cu") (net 41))
 (segment (start 157.48 113.03) (end 176.53 113.03) (width 0.25) (layer "F.Cu") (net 41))
 (segment (start 153.67 83.82) (end 151.13 81.28) (width 0.25) (layer "F.Cu") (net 41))
 (segment (start 154.94 107.95) (end 158.75 111.76) (width 0.25) (layer "F.Cu") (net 42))
 (segment (start 176.53 104.14) (end 182.88 97.79) (width 0.25) (layer "F.Cu") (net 42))
 (segment (start 152.408888 78.748888) (end 152.4 78.757776) (width 0.25) (layer "F.Cu") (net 42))
 (segment (start 176.53 109.22) (end 176.53 104.14) (width 0.25) (layer "F.Cu") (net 42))
 (segment (start 154.94 81.28) (end 154.94 107.95) (width 0.25) (layer "F.Cu") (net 42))
 (segment (start 152.4 78.757776) (end 152.391112 78.748888) (width 0.25) (layer "F.Cu") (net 42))
 (segment (start 152.408888 78.748888) (end 154.94 81.28) (width 0.25) (layer "F.Cu") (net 42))
 (segment (start 152.391112 78.748888) (end 143.5 78.748888) (width 0.25) (layer "F.Cu") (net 42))
 (segment (start 158.75 111.76) (end 173.99 111.76) (width 0.25) (layer "F.Cu") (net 42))
 (segment (start 173.99 111.76) (end 176.53 109.22) (width 0.25) (layer "F.Cu") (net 42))
 (segment (start 182.88 97.79) (end 185.99 97.79) (width 0.25) (layer "F.Cu") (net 42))
 (segment (start 144.777768 104.137768) (end 143.5 104.137768) (width 0.25) (layer "F.Cu") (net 32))
 (segment (start 156.94 120.65) (end 155.67 121.92) (width 0.25) (layer "F.Cu") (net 32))
 (segment (start 146.05 105.41) (end 144.777768 104.137768) (width 0.25) (layer "F.Cu") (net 32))
 (segment (start 155.67 121.92) (end 152.4 121.92) (width 0.25) (layer "F.Cu") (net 32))
 (segment (start 152.4 121.92) (end 146.05 115.57) (width 0.25) (layer "F.Cu") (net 32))
 (segment (start 146.05 115.57) (end 146.05 105.41) (width 0.25) (layer "F.Cu") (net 32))
 (segment (start 146.04888 101.59888) (end 143.5 101.59888) (width 0.25) (layer "F.Cu") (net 33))
 (segment (start 154.94 120.65) (end 153.67 120.65) (width 0.25) (layer "F.Cu") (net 33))
 (segment (start 147.32 102.87) (end 146.04888 101.59888) (width 0.25) (layer "F.Cu") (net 33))
 (segment (start 153.67 120.65) (end 147.32 114.3) (width 0.25) (layer "F.Cu") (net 33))
 (segment (start 147.32 114.3) (end 147.32 102.87) (width 0.25) (layer "F.Cu") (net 33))
 (segment (start 85.74 92.41) (end 85.74 97.72) (width 0.25) (layer "F.Cu") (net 5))
 (segment (start 71.36 78.03) (end 85.74 92.41) (width 0.25) (layer "F.Cu") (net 5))
 (segment (start 71.74 97.72) (end 71.74 84.91) (width 0.25) (layer "F.Cu") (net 6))
 (segment (start 71.74 84.91) (end 71.36 84.53) (width 0.25) (layer "F.Cu") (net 6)))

